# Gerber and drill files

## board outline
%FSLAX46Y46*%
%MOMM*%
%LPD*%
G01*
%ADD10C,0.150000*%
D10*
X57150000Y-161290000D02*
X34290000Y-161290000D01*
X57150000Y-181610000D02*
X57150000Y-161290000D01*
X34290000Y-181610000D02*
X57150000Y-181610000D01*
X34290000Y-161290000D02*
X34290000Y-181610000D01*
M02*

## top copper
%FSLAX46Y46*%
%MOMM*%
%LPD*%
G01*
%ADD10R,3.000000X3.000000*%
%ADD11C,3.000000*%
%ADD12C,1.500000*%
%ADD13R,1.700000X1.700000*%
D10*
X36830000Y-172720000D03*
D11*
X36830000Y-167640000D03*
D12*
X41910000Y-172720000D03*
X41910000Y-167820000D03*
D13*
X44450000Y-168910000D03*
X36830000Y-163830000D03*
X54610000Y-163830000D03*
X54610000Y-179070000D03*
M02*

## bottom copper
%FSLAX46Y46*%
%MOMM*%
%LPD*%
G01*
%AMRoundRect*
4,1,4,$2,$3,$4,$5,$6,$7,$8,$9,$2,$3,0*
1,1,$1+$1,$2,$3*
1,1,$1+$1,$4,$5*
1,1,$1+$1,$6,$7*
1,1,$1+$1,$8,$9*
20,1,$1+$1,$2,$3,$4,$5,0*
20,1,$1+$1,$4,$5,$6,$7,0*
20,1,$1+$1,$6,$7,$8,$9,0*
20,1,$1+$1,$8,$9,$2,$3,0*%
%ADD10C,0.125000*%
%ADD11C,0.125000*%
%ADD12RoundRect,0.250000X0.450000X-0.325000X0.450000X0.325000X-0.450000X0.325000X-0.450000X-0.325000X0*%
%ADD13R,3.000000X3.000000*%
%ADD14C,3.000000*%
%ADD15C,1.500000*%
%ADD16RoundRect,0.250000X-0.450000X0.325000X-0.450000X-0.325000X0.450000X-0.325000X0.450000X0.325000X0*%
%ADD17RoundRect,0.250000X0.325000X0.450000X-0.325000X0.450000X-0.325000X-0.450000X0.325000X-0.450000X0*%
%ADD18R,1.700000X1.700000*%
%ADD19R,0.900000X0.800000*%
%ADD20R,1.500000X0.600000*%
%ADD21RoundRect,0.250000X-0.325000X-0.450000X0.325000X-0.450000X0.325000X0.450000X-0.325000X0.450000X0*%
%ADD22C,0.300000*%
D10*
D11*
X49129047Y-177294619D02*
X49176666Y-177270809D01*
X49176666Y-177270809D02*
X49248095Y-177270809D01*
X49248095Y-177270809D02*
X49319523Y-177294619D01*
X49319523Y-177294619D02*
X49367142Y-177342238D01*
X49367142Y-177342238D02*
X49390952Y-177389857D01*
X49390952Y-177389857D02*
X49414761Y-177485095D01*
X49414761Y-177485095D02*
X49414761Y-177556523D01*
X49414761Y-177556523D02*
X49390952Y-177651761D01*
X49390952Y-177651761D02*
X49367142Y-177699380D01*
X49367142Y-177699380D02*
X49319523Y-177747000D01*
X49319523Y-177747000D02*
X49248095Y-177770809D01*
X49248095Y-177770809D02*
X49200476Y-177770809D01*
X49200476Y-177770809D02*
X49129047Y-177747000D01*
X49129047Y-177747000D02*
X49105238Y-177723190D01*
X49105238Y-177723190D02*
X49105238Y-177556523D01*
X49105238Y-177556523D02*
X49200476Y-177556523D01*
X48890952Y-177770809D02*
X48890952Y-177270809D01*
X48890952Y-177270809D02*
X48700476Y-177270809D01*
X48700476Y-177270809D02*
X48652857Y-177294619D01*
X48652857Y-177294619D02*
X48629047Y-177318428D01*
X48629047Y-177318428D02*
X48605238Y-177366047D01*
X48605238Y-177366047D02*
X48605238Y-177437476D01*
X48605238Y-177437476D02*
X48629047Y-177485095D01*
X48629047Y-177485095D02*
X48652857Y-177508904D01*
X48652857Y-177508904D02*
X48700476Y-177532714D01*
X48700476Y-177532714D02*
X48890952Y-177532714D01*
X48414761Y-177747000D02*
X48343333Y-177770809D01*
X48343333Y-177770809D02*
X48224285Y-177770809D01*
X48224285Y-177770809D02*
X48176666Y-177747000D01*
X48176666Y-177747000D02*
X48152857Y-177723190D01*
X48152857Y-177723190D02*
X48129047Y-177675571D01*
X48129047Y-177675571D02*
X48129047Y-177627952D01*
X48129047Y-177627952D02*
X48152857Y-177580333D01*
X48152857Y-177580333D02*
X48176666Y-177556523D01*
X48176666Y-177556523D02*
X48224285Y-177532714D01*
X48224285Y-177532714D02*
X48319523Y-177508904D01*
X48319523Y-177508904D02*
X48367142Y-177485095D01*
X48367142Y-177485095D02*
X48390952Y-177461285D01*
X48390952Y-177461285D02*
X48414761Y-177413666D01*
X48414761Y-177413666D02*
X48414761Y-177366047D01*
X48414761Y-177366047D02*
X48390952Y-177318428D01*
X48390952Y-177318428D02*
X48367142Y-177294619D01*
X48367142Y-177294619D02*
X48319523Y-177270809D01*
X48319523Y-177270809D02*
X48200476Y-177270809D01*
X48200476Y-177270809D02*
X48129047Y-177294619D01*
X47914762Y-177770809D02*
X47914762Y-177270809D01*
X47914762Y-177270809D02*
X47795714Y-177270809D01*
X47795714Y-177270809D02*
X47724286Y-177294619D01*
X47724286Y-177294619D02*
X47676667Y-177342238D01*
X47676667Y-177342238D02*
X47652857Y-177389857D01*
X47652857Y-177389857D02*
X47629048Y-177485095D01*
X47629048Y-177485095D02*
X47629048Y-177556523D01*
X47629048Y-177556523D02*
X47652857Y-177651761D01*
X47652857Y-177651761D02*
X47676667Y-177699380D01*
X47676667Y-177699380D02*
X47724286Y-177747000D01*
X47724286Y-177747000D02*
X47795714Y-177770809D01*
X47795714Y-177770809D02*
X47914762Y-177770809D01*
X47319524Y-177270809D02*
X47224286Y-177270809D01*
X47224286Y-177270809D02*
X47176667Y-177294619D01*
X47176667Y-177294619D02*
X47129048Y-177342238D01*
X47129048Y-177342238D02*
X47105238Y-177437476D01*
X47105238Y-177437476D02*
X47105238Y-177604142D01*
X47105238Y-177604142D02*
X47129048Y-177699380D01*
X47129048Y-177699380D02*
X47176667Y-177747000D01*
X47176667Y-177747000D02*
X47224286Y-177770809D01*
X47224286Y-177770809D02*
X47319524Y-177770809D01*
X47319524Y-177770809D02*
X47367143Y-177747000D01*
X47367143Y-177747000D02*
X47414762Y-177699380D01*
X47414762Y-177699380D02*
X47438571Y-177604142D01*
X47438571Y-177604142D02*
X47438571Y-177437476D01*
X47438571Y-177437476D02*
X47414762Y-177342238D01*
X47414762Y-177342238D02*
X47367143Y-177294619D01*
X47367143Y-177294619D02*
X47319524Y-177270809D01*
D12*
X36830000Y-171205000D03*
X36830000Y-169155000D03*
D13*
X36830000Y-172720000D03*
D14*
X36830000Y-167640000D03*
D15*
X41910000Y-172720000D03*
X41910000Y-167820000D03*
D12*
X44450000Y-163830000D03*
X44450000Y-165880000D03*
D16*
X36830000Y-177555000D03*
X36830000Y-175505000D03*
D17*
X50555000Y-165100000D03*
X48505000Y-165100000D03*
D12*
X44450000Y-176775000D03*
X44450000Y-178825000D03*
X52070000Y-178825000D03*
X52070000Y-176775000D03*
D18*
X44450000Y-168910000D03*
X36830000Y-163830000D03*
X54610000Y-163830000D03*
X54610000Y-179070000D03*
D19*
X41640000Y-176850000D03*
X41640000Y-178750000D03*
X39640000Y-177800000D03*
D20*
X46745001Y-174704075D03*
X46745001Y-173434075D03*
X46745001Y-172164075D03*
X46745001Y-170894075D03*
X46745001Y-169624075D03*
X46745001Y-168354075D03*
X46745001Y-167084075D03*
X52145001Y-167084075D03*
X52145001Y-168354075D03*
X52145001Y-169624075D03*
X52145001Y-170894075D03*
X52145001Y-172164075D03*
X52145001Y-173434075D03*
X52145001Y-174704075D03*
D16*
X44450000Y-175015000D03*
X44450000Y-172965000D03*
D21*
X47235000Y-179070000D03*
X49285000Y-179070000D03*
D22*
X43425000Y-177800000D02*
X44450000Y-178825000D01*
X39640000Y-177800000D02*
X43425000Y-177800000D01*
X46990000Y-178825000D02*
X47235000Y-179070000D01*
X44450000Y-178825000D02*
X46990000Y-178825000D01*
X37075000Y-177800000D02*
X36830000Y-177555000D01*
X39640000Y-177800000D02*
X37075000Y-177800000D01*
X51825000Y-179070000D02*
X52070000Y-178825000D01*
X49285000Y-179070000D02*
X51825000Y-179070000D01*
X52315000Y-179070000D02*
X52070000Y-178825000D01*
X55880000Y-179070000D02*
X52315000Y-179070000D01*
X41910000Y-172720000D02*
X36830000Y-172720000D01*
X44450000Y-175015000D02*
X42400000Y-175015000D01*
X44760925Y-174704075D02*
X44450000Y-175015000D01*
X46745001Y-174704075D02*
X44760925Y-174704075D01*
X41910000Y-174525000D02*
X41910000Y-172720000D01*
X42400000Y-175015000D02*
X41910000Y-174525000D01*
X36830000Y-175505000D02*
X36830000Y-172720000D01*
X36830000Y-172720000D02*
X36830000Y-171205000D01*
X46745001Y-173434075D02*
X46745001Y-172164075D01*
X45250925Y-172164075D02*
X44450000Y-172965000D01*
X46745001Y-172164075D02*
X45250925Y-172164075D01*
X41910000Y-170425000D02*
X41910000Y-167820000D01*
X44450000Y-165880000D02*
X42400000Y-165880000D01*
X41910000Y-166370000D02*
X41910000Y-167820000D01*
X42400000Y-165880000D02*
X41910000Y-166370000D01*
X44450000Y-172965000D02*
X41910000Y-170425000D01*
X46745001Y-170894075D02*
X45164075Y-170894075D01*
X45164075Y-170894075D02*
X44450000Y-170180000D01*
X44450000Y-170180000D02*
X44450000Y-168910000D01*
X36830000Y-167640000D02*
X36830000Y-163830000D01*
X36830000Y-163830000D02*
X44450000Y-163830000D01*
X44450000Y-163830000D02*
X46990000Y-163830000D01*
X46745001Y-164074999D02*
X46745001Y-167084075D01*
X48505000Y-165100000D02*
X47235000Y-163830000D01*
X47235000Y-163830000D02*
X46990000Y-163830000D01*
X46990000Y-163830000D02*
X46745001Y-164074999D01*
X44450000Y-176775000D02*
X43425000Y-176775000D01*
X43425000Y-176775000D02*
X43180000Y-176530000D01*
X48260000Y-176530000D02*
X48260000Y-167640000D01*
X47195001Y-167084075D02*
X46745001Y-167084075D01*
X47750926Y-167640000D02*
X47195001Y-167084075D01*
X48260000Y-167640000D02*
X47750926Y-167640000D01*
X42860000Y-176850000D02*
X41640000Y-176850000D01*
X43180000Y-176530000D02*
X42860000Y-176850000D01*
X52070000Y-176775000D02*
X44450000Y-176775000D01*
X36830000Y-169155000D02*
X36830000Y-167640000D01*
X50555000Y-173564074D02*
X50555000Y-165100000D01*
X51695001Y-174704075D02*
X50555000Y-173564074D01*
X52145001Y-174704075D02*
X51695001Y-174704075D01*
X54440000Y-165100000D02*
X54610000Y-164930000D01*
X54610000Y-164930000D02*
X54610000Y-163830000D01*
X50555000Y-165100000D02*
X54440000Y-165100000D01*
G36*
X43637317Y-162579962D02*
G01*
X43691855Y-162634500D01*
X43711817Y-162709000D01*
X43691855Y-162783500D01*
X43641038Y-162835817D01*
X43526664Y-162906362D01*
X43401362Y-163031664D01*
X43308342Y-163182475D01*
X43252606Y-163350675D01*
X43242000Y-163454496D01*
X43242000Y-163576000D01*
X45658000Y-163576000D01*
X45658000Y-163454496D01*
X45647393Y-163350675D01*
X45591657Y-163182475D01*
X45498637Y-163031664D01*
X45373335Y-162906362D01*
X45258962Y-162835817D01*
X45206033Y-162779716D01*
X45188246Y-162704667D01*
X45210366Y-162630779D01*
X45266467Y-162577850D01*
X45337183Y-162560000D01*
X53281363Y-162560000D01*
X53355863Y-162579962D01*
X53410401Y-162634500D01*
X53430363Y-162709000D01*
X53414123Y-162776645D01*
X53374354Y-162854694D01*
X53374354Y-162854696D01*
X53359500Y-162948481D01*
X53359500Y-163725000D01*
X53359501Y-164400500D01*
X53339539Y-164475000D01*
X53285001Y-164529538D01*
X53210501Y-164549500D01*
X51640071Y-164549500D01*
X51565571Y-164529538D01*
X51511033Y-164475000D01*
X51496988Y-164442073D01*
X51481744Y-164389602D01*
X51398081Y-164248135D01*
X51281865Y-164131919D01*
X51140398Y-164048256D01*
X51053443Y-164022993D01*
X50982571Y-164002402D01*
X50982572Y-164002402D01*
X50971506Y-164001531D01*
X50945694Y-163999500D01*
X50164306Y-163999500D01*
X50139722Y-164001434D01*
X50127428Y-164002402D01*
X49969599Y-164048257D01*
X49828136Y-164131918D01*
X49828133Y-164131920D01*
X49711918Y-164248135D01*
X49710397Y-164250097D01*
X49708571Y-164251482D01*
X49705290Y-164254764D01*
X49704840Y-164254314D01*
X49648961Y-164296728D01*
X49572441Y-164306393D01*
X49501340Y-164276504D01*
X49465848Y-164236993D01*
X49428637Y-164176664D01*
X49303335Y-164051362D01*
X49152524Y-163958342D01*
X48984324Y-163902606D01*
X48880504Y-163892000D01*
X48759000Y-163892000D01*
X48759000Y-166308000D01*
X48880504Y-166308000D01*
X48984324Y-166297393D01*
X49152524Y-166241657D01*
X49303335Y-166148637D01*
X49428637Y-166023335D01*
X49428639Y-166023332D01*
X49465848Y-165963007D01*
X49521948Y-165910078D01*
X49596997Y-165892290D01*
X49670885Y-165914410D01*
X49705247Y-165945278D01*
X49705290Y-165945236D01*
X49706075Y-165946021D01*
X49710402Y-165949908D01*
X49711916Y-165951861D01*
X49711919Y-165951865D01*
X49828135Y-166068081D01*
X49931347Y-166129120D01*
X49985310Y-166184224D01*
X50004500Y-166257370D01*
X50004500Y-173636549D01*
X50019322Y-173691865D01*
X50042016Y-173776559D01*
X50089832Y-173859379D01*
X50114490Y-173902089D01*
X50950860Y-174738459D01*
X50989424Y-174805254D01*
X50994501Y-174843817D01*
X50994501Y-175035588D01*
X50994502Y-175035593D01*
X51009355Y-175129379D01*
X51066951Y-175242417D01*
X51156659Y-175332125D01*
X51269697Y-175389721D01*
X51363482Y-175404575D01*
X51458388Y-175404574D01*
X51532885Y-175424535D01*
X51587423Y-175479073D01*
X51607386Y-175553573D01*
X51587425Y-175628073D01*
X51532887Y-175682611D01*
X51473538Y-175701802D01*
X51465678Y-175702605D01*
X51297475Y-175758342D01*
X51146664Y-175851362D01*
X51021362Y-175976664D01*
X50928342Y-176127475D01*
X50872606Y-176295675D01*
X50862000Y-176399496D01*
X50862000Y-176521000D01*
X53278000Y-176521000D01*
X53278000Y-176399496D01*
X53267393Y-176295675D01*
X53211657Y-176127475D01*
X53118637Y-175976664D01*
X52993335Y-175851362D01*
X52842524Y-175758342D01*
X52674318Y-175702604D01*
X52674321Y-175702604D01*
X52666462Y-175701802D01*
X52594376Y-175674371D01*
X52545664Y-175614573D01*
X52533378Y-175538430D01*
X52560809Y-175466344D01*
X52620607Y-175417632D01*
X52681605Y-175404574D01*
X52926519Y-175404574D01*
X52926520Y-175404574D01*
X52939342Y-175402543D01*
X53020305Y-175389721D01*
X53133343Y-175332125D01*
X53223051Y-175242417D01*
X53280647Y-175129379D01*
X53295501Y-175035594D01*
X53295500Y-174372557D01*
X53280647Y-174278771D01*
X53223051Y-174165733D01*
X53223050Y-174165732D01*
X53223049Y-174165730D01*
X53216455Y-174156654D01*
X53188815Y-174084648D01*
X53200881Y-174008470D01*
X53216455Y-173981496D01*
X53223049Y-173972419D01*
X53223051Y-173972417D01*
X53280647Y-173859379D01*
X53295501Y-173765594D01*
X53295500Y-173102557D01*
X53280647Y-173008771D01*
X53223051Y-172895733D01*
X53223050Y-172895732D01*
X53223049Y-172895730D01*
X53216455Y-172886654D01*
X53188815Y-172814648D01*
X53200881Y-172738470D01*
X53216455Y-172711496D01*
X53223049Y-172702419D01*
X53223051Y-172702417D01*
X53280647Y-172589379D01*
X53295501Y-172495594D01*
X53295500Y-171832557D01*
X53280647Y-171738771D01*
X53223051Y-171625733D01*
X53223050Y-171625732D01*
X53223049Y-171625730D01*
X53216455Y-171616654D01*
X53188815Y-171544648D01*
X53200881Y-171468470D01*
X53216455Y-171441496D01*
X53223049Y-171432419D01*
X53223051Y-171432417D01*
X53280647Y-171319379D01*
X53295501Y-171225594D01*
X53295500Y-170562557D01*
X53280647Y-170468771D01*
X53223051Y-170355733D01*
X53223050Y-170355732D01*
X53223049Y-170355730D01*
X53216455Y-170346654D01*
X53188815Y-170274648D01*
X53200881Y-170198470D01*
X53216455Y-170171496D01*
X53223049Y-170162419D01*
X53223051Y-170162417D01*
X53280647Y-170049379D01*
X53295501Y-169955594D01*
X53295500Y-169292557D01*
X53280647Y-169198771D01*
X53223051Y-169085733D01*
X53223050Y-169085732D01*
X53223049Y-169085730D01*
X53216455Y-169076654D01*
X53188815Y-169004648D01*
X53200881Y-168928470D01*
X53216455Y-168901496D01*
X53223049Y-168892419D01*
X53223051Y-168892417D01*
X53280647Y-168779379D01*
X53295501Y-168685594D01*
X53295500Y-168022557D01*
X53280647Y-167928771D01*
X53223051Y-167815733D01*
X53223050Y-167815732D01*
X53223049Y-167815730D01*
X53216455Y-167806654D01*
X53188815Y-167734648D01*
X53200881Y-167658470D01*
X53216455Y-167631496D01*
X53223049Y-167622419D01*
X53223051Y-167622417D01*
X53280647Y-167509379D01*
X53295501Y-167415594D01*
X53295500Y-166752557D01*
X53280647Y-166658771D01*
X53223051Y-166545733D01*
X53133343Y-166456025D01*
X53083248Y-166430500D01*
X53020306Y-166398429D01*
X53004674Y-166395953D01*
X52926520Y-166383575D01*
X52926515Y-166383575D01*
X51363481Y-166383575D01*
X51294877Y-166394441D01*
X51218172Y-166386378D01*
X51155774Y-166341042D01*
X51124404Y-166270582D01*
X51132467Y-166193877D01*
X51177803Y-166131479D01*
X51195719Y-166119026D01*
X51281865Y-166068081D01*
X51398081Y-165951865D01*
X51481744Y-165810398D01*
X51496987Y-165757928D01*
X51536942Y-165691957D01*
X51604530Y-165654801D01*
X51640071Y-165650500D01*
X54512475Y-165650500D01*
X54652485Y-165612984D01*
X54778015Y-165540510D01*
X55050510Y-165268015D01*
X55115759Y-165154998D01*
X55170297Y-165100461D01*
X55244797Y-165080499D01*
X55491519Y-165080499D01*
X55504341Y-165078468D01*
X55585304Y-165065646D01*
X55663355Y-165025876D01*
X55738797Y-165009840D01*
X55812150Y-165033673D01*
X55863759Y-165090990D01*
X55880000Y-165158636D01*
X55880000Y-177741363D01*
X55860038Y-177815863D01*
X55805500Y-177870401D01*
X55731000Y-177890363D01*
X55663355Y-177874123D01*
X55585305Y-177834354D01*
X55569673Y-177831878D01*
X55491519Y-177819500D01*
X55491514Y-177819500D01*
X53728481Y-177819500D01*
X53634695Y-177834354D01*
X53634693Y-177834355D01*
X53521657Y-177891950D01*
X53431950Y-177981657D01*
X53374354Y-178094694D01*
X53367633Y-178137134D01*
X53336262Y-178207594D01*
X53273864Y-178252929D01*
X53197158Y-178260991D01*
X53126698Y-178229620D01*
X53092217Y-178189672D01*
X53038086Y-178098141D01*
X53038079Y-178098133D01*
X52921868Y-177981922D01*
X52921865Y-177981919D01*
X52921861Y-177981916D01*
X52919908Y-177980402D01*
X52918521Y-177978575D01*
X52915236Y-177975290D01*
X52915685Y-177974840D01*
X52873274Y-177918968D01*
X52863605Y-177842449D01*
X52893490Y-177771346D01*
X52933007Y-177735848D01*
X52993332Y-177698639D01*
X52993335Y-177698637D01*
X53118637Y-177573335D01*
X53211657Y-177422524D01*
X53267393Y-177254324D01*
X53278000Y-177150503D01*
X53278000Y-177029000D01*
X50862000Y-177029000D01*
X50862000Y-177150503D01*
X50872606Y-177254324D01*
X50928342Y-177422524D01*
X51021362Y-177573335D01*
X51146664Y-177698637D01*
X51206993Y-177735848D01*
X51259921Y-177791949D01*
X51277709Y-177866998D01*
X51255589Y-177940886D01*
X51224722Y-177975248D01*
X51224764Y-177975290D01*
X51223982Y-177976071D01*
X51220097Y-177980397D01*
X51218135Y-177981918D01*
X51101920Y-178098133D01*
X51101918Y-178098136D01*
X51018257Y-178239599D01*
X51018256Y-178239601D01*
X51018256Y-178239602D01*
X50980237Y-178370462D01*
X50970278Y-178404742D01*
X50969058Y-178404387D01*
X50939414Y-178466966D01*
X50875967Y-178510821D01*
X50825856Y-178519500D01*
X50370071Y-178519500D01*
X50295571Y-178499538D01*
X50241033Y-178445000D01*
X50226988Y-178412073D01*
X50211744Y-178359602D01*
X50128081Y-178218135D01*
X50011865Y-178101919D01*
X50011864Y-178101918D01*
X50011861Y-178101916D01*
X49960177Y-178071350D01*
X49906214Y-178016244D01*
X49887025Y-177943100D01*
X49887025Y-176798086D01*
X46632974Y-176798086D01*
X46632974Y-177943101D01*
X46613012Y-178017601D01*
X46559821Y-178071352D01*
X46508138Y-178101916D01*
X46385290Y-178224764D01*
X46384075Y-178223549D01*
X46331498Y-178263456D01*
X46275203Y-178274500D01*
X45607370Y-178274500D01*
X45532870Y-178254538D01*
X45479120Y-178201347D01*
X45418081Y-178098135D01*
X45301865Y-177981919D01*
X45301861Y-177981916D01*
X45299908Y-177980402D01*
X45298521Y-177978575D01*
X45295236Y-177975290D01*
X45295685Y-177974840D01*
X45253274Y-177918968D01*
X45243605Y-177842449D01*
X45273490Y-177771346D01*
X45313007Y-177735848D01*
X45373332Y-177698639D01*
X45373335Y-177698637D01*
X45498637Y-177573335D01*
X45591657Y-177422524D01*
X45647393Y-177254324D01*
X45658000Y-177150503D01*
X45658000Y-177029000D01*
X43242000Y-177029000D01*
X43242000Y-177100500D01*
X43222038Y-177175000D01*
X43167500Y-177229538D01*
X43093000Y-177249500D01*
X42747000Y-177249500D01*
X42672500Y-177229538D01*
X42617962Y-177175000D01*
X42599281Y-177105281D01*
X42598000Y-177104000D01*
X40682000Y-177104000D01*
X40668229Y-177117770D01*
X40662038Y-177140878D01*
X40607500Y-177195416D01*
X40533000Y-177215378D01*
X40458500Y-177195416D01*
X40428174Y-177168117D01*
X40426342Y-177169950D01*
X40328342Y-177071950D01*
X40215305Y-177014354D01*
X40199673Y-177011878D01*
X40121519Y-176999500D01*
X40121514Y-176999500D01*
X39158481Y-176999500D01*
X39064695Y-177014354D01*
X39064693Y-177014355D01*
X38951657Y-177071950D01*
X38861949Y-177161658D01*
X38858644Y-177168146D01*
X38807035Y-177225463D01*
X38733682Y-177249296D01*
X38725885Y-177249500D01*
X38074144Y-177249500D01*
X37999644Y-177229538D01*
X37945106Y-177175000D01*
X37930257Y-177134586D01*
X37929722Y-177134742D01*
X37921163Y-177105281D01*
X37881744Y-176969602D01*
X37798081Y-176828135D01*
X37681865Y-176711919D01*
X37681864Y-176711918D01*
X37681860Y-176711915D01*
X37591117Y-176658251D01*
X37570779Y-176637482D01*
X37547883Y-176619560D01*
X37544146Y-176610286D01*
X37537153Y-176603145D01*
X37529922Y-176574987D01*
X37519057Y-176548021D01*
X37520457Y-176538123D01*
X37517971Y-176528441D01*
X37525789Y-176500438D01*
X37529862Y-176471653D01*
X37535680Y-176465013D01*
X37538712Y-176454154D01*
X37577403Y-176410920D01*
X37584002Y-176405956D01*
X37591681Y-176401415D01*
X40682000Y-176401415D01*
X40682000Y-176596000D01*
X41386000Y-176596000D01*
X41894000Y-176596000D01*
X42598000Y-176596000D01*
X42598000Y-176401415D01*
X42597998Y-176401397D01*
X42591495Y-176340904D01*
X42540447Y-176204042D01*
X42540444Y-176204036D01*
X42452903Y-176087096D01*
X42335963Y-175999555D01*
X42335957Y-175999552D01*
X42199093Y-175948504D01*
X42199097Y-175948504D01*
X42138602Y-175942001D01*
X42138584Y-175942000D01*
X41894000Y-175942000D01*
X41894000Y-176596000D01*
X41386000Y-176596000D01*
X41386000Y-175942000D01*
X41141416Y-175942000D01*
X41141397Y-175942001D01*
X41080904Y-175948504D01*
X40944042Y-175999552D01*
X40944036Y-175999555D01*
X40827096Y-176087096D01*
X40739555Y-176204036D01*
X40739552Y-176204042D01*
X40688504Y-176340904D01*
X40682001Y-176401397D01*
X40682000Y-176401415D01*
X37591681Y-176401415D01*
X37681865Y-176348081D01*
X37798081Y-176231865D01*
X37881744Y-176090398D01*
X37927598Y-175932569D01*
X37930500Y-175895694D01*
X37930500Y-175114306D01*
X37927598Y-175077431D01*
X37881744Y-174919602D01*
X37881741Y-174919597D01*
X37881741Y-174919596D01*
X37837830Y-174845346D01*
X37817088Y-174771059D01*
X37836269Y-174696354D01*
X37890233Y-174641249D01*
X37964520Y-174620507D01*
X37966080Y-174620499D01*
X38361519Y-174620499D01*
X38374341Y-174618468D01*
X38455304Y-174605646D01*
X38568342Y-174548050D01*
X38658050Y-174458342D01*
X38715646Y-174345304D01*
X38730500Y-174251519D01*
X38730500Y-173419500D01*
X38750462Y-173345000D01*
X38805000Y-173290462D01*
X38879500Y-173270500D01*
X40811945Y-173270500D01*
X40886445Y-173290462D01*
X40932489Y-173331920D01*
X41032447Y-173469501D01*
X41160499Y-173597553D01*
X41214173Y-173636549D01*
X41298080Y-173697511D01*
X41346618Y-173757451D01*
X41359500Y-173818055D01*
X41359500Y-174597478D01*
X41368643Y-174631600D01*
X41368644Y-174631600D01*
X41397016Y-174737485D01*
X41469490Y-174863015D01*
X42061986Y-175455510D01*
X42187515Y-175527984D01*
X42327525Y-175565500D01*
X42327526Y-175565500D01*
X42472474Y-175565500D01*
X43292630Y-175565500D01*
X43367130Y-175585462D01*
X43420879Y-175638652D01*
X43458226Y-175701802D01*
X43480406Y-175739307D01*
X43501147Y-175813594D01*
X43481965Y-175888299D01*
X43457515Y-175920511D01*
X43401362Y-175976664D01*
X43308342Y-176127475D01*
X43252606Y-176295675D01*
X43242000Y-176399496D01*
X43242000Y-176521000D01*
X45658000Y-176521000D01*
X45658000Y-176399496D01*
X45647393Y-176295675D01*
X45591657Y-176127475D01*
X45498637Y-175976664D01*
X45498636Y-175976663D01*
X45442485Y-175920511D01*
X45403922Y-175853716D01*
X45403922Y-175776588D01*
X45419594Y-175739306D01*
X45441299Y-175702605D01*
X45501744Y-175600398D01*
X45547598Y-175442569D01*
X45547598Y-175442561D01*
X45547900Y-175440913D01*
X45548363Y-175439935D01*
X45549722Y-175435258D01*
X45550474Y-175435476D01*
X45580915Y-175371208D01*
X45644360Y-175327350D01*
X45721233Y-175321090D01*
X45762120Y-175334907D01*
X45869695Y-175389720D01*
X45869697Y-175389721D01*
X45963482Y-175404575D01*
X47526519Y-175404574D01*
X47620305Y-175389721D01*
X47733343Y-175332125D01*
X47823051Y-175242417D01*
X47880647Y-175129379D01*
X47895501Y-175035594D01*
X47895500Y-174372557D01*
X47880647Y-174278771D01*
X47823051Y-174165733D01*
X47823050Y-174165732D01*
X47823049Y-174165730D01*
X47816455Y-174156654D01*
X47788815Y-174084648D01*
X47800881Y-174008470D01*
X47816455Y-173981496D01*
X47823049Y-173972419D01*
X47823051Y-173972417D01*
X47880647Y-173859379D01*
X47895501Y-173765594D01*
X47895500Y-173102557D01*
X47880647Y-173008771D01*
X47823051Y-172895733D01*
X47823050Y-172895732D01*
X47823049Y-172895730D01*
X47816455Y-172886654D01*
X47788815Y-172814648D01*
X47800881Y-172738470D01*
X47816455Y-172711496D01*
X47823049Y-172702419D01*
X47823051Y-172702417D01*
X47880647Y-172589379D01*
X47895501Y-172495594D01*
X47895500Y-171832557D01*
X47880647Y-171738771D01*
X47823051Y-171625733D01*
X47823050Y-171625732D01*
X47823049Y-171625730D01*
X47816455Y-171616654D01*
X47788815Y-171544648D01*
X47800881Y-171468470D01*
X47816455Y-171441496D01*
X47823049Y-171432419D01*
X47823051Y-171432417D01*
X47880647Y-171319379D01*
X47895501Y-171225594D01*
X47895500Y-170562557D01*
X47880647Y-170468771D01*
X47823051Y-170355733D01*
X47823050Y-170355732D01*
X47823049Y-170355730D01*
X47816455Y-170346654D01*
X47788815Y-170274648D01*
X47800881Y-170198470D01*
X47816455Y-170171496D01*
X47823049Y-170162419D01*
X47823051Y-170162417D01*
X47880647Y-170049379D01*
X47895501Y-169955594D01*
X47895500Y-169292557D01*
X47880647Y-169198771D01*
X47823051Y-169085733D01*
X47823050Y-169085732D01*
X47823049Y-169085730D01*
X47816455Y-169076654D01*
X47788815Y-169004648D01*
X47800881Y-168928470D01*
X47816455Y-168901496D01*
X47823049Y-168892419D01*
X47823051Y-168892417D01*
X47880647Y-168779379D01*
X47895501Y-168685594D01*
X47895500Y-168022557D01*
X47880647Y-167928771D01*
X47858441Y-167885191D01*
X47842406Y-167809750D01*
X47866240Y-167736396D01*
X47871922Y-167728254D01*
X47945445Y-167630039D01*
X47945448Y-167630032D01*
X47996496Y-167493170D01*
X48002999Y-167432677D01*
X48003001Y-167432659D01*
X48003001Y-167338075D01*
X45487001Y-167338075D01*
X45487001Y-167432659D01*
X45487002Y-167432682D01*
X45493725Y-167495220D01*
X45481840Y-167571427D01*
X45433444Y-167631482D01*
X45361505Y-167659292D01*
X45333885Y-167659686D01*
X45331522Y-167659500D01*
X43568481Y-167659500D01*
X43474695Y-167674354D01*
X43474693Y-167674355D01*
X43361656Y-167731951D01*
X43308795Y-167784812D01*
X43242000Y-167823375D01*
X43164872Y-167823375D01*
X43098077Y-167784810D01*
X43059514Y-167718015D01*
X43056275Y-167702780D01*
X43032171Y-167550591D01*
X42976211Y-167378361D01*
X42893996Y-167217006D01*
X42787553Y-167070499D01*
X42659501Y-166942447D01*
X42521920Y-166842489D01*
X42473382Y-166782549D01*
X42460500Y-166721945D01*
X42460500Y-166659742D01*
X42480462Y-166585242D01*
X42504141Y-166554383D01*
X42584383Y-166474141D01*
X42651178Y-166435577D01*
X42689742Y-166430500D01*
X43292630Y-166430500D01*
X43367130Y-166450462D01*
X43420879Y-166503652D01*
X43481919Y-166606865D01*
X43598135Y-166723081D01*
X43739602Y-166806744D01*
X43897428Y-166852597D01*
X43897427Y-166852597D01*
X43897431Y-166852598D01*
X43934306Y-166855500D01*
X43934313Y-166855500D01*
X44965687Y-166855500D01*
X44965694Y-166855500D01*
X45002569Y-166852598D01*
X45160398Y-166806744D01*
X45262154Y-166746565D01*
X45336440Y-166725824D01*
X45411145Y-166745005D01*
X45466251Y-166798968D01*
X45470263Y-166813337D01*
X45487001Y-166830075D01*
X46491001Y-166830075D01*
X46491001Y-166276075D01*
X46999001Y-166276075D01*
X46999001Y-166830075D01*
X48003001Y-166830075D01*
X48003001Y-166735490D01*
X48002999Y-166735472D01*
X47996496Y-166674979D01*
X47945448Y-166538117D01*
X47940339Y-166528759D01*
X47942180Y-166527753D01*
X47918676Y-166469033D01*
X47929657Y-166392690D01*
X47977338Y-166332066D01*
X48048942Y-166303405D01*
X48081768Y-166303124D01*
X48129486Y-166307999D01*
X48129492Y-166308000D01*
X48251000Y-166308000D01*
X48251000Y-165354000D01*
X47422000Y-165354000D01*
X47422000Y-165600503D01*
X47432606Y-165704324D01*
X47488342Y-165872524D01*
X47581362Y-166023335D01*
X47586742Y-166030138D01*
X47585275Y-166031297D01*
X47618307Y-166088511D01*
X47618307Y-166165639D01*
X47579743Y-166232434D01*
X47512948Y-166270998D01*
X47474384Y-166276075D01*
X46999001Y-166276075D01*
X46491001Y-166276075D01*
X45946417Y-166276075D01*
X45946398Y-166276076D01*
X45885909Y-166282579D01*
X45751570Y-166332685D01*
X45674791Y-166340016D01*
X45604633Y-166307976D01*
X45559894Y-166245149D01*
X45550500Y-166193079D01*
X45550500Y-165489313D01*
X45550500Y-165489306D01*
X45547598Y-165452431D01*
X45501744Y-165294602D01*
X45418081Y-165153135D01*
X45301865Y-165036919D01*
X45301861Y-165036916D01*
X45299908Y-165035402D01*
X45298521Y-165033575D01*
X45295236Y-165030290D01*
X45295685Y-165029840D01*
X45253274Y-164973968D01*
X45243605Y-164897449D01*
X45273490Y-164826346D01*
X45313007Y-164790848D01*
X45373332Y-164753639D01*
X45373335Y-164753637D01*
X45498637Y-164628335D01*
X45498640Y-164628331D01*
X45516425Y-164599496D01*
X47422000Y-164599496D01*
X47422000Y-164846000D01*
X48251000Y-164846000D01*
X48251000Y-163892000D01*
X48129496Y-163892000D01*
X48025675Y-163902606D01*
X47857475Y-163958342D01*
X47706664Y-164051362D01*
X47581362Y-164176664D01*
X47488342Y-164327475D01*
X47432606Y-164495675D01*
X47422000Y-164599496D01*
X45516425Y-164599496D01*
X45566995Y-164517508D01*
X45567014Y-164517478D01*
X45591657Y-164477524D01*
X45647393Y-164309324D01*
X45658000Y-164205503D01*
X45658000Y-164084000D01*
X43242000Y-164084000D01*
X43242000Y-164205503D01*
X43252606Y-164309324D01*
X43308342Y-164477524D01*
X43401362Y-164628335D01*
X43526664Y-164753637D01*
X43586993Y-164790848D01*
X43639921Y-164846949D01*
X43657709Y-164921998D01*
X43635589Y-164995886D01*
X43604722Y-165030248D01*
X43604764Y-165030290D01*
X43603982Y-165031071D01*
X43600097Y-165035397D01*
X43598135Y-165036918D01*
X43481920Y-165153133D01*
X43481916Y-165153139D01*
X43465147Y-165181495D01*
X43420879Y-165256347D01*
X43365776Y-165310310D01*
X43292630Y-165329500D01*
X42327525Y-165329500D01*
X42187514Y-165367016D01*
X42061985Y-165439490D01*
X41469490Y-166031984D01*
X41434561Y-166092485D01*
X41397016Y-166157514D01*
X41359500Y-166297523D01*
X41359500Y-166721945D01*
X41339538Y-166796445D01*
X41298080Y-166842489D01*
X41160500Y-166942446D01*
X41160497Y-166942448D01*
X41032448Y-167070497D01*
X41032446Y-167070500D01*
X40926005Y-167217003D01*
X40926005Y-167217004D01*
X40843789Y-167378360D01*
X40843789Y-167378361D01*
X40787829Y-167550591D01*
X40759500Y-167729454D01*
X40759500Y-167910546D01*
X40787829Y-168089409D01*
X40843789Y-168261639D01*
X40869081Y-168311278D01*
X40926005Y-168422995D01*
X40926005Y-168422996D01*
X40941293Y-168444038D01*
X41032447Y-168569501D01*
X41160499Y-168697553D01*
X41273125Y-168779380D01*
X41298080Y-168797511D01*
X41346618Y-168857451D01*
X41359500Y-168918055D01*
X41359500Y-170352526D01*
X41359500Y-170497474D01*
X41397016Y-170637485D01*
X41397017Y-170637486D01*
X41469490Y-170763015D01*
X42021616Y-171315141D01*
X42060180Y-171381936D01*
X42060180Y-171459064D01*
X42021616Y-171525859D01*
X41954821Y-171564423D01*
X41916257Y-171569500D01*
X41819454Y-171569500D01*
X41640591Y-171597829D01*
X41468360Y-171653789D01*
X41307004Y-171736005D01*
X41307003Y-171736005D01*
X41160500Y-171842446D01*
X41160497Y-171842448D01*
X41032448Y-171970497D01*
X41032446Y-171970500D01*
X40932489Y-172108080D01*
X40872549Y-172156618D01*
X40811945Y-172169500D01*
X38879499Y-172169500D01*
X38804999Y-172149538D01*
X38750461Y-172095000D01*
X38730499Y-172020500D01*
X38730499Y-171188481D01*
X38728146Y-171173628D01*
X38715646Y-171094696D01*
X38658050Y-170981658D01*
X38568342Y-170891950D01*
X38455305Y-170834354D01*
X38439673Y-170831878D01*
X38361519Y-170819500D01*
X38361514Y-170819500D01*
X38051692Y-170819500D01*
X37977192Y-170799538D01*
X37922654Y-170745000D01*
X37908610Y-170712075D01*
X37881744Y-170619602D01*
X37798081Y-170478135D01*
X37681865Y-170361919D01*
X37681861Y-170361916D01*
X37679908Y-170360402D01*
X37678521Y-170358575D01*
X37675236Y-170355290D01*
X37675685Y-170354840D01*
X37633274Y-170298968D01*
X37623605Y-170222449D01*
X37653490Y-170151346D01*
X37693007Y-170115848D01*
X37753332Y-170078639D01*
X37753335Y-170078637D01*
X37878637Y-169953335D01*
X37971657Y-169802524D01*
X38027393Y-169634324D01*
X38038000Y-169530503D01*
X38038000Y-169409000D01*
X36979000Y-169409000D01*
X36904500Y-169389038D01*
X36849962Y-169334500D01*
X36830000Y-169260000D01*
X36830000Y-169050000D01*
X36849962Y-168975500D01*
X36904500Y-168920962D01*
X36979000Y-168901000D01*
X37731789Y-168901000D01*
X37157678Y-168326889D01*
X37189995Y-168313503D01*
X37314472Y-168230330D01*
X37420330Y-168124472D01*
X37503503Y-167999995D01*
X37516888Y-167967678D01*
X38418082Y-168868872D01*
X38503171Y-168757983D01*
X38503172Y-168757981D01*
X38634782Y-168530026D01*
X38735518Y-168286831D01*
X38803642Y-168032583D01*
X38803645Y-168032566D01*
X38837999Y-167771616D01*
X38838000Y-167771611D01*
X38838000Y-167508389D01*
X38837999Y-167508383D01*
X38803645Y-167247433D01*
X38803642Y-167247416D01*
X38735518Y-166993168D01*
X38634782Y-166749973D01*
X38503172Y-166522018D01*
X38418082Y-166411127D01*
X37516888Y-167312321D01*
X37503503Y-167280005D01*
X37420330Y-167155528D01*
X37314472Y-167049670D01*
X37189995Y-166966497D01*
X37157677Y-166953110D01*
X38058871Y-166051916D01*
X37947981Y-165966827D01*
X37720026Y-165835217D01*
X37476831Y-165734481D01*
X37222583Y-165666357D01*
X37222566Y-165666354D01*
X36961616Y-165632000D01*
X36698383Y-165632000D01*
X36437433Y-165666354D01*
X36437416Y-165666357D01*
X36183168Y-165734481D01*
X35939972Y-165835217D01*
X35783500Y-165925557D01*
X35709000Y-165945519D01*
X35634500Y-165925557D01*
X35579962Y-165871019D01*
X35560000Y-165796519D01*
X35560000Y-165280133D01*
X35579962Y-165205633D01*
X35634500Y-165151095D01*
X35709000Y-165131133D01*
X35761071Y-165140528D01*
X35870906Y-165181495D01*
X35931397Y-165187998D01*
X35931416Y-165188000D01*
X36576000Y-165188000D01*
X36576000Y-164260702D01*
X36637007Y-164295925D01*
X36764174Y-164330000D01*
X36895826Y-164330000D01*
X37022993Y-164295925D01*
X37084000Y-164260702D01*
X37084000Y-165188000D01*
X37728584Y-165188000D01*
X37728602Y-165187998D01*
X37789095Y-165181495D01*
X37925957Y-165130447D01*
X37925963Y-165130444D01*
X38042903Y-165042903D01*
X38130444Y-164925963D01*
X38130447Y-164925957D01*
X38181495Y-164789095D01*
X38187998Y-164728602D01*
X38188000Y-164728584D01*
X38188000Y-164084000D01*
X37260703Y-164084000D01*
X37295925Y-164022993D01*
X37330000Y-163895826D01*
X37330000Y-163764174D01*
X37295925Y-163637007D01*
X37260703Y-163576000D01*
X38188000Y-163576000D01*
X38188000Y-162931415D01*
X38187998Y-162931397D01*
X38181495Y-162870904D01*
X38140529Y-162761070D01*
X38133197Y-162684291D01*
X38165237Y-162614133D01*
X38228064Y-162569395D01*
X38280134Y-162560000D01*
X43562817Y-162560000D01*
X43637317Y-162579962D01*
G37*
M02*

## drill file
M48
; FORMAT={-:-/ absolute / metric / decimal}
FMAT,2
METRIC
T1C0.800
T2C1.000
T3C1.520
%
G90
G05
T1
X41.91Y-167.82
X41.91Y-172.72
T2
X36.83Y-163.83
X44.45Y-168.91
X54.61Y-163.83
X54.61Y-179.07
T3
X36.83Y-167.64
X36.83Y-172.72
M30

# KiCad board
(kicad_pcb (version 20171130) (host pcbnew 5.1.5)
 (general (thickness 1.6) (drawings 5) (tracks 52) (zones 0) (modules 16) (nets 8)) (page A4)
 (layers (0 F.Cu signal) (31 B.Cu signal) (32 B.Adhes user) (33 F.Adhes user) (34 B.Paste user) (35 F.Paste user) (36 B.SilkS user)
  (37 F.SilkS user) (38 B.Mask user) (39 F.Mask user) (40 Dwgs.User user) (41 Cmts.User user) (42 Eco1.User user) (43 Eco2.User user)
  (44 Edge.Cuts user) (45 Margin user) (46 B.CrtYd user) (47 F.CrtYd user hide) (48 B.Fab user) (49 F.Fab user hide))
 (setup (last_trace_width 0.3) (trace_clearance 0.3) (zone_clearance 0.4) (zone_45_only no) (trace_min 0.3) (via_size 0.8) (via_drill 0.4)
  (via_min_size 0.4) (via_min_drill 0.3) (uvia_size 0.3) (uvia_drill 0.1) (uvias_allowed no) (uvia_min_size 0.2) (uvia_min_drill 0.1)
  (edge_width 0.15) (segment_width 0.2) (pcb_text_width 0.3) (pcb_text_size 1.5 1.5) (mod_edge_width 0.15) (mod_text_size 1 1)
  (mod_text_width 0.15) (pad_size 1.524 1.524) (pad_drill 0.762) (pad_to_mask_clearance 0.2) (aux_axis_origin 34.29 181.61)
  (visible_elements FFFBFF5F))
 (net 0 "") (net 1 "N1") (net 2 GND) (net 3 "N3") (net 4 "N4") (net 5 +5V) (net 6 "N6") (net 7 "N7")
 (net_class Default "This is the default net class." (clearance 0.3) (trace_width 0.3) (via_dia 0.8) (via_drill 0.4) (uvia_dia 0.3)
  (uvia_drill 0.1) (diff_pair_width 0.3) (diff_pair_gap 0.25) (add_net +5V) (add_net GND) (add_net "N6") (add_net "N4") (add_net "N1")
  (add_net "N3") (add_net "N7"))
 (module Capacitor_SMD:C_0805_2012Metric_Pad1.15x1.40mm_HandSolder (layer B.Cu) (at 36.83 170.18 90)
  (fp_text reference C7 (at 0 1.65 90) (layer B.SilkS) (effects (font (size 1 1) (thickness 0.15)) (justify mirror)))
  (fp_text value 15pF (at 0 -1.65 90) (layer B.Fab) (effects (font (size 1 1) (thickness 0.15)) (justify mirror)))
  (pad 1 smd roundrect (at -1.025 0 90) (size 1.15 1.4) (layers B.Cu B.Paste B.Mask) (roundrect_rratio 0.217391) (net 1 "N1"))
  (pad 2 smd roundrect (at 1.025 0 90) (size 1.15 1.4) (layers B.Cu B.Paste B.Mask) (roundrect_rratio 0.217391) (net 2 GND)))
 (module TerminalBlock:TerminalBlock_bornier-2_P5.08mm (layer B.Cu) (at 36.83 172.72 90)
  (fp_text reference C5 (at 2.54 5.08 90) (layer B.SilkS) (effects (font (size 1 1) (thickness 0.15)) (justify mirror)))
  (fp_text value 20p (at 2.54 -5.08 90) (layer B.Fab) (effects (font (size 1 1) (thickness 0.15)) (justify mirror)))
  (pad 1 thru_hole rect (at 0 0 90) (size 3 3) (drill 1.52) (layers *.Cu *.Mask) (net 1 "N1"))
  (pad 2 thru_hole circle (at 5.08 0 90) (size 3 3) (drill 1.52) (layers *.Cu *.Mask) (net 2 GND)))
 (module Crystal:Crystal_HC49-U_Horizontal (layer F.Cu) (at 41.91 172.72 90)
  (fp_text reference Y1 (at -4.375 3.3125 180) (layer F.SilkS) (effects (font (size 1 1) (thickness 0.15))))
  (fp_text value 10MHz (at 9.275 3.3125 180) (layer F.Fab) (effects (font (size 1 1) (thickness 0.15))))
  (pad 1 thru_hole circle (at 0 0 90) (size 1.5 1.5) (drill 0.8) (layers *.Cu *.Mask) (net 1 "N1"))
  (pad 2 thru_hole circle (at 4.9 0 90) (size 1.5 1.5) (drill 0.8) (layers *.Cu *.Mask) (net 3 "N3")))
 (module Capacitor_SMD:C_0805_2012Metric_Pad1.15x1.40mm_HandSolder (layer B.Cu) (at 44.45 164.855 90)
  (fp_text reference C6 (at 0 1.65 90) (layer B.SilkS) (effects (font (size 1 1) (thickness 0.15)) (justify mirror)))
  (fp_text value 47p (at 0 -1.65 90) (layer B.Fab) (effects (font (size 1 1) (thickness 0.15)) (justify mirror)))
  (pad 2 smd roundrect (at 1.025 0 90) (size 1.15 1.4) (layers B.Cu B.Paste B.Mask) (roundrect_rratio 0.217391) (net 2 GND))
  (pad 1 smd roundrect (at -1.025 0 90) (size 1.15 1.4) (layers B.Cu B.Paste B.Mask) (roundrect_rratio 0.217391) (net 3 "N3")))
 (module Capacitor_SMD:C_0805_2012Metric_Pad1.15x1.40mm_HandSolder (layer B.Cu) (at 36.83 176.53 270)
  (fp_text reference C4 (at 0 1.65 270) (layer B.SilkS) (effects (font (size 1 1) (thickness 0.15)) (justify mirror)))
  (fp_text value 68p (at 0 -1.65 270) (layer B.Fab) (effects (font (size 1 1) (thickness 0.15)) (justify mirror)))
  (pad 2 smd roundrect (at 1.025 0 270) (size 1.15 1.4) (layers B.Cu B.Paste B.Mask) (roundrect_rratio 0.217391) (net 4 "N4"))
  (pad 1 smd roundrect (at -1.025 0 270) (size 1.15 1.4) (layers B.Cu B.Paste B.Mask) (roundrect_rratio 0.217391) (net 1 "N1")))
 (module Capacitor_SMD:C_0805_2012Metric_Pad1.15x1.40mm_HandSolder (layer B.Cu) (at 49.53 165.1 180)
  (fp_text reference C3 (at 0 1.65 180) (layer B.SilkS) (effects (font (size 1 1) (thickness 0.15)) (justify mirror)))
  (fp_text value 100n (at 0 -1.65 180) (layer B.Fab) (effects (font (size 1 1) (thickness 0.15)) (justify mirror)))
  (pad 1 smd roundrect (at -1.025 0 180) (size 1.15 1.4) (layers B.Cu B.Paste B.Mask) (roundrect_rratio 0.217391) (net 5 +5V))
  (pad 2 smd roundrect (at 1.025 0 180) (size 1.15 1.4) (layers B.Cu B.Paste B.Mask) (roundrect_rratio 0.217391) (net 2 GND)))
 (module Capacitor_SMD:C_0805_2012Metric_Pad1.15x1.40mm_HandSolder (layer B.Cu) (at 44.45 177.8 90)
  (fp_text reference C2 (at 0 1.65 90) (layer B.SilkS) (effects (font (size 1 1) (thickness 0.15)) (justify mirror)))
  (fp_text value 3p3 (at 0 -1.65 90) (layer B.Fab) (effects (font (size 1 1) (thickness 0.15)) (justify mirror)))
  (pad 2 smd roundrect (at 1.025 0 90) (size 1.15 1.4) (layers B.Cu B.Paste B.Mask) (roundrect_rratio 0.217391) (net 2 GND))
  (pad 1 smd roundrect (at -1.025 0 90) (size 1.15 1.4) (layers B.Cu B.Paste B.Mask) (roundrect_rratio 0.217391) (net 4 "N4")))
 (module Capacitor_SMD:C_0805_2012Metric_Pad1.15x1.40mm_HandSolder (layer B.Cu) (at 52.07 177.8 90)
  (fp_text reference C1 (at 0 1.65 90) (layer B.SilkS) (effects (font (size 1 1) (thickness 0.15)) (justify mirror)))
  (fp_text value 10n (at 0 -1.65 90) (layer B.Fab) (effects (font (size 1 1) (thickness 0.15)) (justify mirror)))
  (pad 1 smd roundrect (at -1.025 0 90) (size 1.15 1.4) (layers B.Cu B.Paste B.Mask) (roundrect_rratio 0.217391) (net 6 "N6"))
  (pad 2 smd roundrect (at 1.025 0 90) (size 1.15 1.4) (layers B.Cu B.Paste B.Mask) (roundrect_rratio 0.217391) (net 2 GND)))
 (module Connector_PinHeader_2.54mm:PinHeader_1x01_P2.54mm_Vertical (layer F.Cu) (at 44.45 168.91)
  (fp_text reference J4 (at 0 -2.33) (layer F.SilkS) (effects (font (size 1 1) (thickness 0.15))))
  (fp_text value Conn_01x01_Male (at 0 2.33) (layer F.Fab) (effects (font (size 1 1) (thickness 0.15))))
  (pad 1 thru_hole rect (at 0 0) (size 1.7 1.7) (drill 1) (layers *.Cu *.Mask) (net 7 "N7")))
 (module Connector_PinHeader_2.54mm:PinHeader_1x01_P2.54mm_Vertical (layer F.Cu) (at 36.83 163.83)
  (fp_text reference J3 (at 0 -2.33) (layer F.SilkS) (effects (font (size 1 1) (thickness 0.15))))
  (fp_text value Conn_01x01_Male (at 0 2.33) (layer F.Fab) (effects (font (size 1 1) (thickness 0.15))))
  (pad 1 thru_hole rect (at 0 0) (size 1.7 1.7) (drill 1) (layers *.Cu *.Mask) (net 2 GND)))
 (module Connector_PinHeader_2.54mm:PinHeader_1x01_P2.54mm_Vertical (layer F.Cu) (at 54.61 163.83)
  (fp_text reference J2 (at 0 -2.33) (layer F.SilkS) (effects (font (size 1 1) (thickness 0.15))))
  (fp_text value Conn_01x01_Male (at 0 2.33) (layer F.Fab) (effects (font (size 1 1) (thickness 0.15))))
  (pad 1 thru_hole rect (at 0 0) (size 1.7 1.7) (drill 1) (layers *.Cu *.Mask) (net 5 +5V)))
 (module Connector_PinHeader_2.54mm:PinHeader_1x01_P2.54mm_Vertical (layer F.Cu) (at 54.61 179.07)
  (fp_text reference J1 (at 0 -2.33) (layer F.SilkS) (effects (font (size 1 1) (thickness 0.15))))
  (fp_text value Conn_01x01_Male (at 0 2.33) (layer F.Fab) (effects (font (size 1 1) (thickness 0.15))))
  (pad 1 thru_hole rect (at 0 0) (size 1.7 1.7) (drill 1) (layers *.Cu *.Mask) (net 6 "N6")))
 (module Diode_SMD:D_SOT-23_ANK (layer B.Cu) (at 40.64 177.8 180)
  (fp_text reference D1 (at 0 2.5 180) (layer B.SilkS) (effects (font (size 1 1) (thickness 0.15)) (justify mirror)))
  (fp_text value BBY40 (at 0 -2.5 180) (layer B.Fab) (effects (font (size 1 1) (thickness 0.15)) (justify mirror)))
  (pad 2 smd rect (at -1 0.95 180) (size 0.9 0.8) (layers B.Cu B.Paste B.Mask) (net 2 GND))
  (pad "" smd rect (at -1 -0.95 180) (size 0.9 0.8) (layers B.Cu B.Paste B.Mask))
  (pad 1 smd rect (at 1 0 180) (size 0.9 0.8) (layers B.Cu B.Paste B.Mask) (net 4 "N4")))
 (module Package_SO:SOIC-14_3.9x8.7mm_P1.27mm (layer B.Cu) (at 49.445001 170.894075)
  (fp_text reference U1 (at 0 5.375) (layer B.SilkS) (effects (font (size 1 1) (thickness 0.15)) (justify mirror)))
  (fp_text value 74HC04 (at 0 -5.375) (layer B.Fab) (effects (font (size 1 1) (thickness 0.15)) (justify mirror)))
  (pad 1 smd rect (at -2.7 3.81) (size 1.5 0.6) (layers B.Cu B.Paste B.Mask) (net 1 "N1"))
  (pad 2 smd rect (at -2.7 2.54) (size 1.5 0.6) (layers B.Cu B.Paste B.Mask) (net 3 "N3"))
  (pad 3 smd rect (at -2.7 1.27) (size 1.5 0.6) (layers B.Cu B.Paste B.Mask) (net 3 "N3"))
  (pad 4 smd rect (at -2.7 0) (size 1.5 0.6) (layers B.Cu B.Paste B.Mask) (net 7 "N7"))
  (pad 5 smd rect (at -2.7 -1.27) (size 1.5 0.6) (layers B.Cu B.Paste B.Mask))
  (pad 6 smd rect (at -2.7 -2.54) (size 1.5 0.6) (layers B.Cu B.Paste B.Mask))
  (pad 7 smd rect (at -2.7 -3.81) (size 1.5 0.6) (layers B.Cu B.Paste B.Mask) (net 2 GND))
  (pad 8 smd rect (at 2.7 -3.81) (size 1.5 0.6) (layers B.Cu B.Paste B.Mask))
  (pad 9 smd rect (at 2.7 -2.54) (size 1.5 0.6) (layers B.Cu B.Paste B.Mask))
  (pad 10 smd rect (at 2.7 -1.27) (size 1.5 0.6) (layers B.Cu B.Paste B.Mask))
  (pad 11 smd rect (at 2.7 0) (size 1.5 0.6) (layers B.Cu B.Paste B.Mask))
  (pad 12 smd rect (at 2.7 1.27) (size 1.5 0.6) (layers B.Cu B.Paste B.Mask))
  (pad 13 smd rect (at 2.7 2.54) (size 1.5 0.6) (layers B.Cu B.Paste B.Mask))
  (pad 14 smd rect (at 2.7 3.81) (size 1.5 0.6) (layers B.Cu B.Paste B.Mask) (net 5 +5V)))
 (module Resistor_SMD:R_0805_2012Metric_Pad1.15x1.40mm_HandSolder (layer B.Cu) (at 44.45 173.99 270)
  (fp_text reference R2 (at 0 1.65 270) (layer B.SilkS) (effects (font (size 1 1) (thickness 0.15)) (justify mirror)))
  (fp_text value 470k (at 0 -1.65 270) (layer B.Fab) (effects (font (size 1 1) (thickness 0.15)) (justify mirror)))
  (pad 2 smd roundrect (at 1.025 0 270) (size 1.15 1.4) (layers B.Cu B.Paste B.Mask) (roundrect_rratio 0.217391) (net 1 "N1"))
  (pad 1 smd roundrect (at -1.025 0 270) (size 1.15 1.4) (layers B.Cu B.Paste B.Mask) (roundrect_rratio 0.217391) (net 3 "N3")))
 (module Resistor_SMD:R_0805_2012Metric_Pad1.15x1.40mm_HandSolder (layer B.Cu) (at 48.26 179.07)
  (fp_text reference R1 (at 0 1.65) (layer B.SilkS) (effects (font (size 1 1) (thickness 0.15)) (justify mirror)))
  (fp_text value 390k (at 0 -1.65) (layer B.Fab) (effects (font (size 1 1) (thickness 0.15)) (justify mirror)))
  (pad 1 smd roundrect (at -1.025 0) (size 1.15 1.4) (layers B.Cu B.Paste B.Mask) (roundrect_rratio 0.217391) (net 4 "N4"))
  (pad 2 smd roundrect (at 1.025 0) (size 1.15 1.4) (layers B.Cu B.Paste B.Mask) (roundrect_rratio 0.217391) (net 6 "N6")))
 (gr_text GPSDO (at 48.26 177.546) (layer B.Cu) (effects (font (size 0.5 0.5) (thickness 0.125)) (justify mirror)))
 (gr_line (start 57.15 161.29) (end 34.29 161.29) (layer Edge.Cuts) (width 0.15))
 (gr_line (start 57.15 181.61) (end 57.15 161.29) (layer Edge.Cuts) (width 0.15))
 (gr_line (start 34.29 181.61) (end 57.15 181.61) (layer Edge.Cuts) (width 0.15))
 (gr_line (start 34.29 161.29) (end 34.29 181.61) (layer Edge.Cuts) (width 0.15))
 (segment (start 43.425 177.8) (end 44.45 178.825) (width 0.3) (layer B.Cu) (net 4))
 (segment (start 39.64 177.8) (end 43.425 177.8) (width 0.3) (layer B.Cu) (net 4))
 (segment (start 46.99 178.825) (end 47.235 179.07) (width 0.3) (layer B.Cu) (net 4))
 (segment (start 44.45 178.825) (end 46.99 178.825) (width 0.3) (layer B.Cu) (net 4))
 (segment (start 37.075 177.8) (end 36.83 177.555) (width 0.3) (layer B.Cu) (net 4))
 (segment (start 39.64 177.8) (end 37.075 177.8) (width 0.3) (layer B.Cu) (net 4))
 (segment (start 51.825 179.07) (end 52.07 178.825) (width 0.3) (layer B.Cu) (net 6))
 (segment (start 49.285 179.07) (end 51.825 179.07) (width 0.3) (layer B.Cu) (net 6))
 (segment (start 52.315 179.07) (end 52.07 178.825) (width 0.3) (layer B.Cu) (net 6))
 (segment (start 55.88 179.07) (end 52.315 179.07) (width 0.3) (layer B.Cu) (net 6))
 (segment (start 41.91 172.72) (end 36.83 172.72) (width 0.3) (layer B.Cu) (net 1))
 (segment (start 44.45 175.015) (end 42.4 175.015) (width 0.3) (layer B.Cu) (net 1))
 (segment (start 44.760925 174.704075) (end 44.45 175.015) (width 0.3) (layer B.Cu) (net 1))
 (segment (start 46.745001 174.704075) (end 44.760925 174.704075) (width 0.3) (layer B.Cu) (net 1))
 (segment (start 41.91 174.525) (end 41.91 172.72) (width 0.3) (layer B.Cu) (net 1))
 (segment (start 42.4 175.015) (end 41.91 174.525) (width 0.3) (layer B.Cu) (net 1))
 (segment (start 36.83 175.505) (end 36.83 172.72) (width 0.3) (layer B.Cu) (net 1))
 (segment (start 36.83 172.72) (end 36.83 171.205) (width 0.3) (layer B.Cu) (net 1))
 (segment (start 46.745001 173.434075) (end 46.745001 172.164075) (width 0.3) (layer B.Cu) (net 3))
 (segment (start 45.250925 172.164075) (end 44.45 172.965) (width 0.3) (layer B.Cu) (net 3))
 (segment (start 46.745001 172.164075) (end 45.250925 172.164075) (width 0.3) (layer B.Cu) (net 3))
 (segment (start 41.91 170.425) (end 41.91 167.82) (width 0.3) (layer B.Cu) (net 3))
 (segment (start 44.45 165.88) (end 42.4 165.88) (width 0.3) (layer B.Cu) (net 3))
 (segment (start 41.91 166.37) (end 41.91 167.82) (width 0.3) (layer B.Cu) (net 3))
 (segment (start 42.4 165.88) (end 41.91 166.37) (width 0.3) (layer B.Cu) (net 3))
 (segment (start 44.45 172.965) (end 41.91 170.425) (width 0.3) (layer B.Cu) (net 3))
 (segment (start 46.745001 170.894075) (end 45.164075 170.894075) (width 0.3) (layer B.Cu) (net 7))
 (segment (start 45.164075 170.894075) (end 44.45 170.18) (width 0.3) (layer B.Cu) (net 7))
 (segment (start 44.45 170.18) (end 44.45 168.91) (width 0.3) (layer B.Cu) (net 7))
 (segment (start 36.83 167.64) (end 36.83 163.83) (width 0.3) (layer B.Cu) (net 2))
 (segment (start 36.83 163.83) (end 44.45 163.83) (width 0.3) (layer B.Cu) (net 2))
 (segment (start 44.45 163.83) (end 46.99 163.83) (width 0.3) (layer B.Cu) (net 2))
 (segment (start 46.745001 164.074999) (end 46.745001 167.084075) (width 0.3) (layer B.Cu) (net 2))
 (segment (start 48.505 165.1) (end 47.235 163.83) (width 0.3) (layer B.Cu) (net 2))
 (segment (start 47.235 163.83) (end 46.99 163.83) (width 0.3) (layer B.Cu) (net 2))
 (segment (start 46.99 163.83) (end 46.745001 164.074999) (width 0.3) (layer B.Cu) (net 2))
 (segment (start 44.45 176.775) (end 43.425 176.775) (width 0.3) (layer B.Cu) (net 2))
 (segment (start 43.425 176.775) (end 43.18 176.53) (width 0.3) (layer B.Cu) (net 2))
 (segment (start 48.26 176.53) (end 48.26 167.64) (width 0.3) (layer B.Cu) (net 2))
 (segment (start 47.195001 167.084075) (end 46.745001 167.084075) (width 0.3) (layer B.Cu) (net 2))
 (segment (start 47.750926 167.64) (end 47.195001 167.084075) (width 0.3) (layer B.Cu) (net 2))
 (segment (start 48.26 167.64) (end 47.750926 167.64) (width 0.3) (layer B.Cu) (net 2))
 (segment (start 42.86 176.85) (end 41.64 176.85) (width 0.3) (layer B.Cu) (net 2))
 (segment (start 43.18 176.53) (end 42.86 176.85) (width 0.3) (layer B.Cu) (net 2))
 (segment (start 52.07 176.775) (end 44.45 176.775) (width 0.3) (layer B.Cu) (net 2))
 (segment (start 36.83 169.155) (end 36.83 167.64) (width 0.3) (layer B.Cu) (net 2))
 (segment (start 50.555 173.564074) (end 50.555 165.1) (width 0.3) (layer B.Cu) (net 5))
 (segment (start 51.695001 174.704075) (end 50.555 173.564074) (width 0.3) (layer B.Cu) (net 5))
 (segment (start 52.145001 174.704075) (end 51.695001 174.704075) (width 0.3) (layer B.Cu) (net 5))
 (segment (start 54.44 165.1) (end 54.61 164.93) (width 0.3) (layer B.Cu) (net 5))
 (segment (start 54.61 164.93) (end 54.61 163.83) (width 0.3) (layer B.Cu) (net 5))
 (segment (start 50.555 165.1) (end 54.44 165.1) (width 0.3) (layer B.Cu) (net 5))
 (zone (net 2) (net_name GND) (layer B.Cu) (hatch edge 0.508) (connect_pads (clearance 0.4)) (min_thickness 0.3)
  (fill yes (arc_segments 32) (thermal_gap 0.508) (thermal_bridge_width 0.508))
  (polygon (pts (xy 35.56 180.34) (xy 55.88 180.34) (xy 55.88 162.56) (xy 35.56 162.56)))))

